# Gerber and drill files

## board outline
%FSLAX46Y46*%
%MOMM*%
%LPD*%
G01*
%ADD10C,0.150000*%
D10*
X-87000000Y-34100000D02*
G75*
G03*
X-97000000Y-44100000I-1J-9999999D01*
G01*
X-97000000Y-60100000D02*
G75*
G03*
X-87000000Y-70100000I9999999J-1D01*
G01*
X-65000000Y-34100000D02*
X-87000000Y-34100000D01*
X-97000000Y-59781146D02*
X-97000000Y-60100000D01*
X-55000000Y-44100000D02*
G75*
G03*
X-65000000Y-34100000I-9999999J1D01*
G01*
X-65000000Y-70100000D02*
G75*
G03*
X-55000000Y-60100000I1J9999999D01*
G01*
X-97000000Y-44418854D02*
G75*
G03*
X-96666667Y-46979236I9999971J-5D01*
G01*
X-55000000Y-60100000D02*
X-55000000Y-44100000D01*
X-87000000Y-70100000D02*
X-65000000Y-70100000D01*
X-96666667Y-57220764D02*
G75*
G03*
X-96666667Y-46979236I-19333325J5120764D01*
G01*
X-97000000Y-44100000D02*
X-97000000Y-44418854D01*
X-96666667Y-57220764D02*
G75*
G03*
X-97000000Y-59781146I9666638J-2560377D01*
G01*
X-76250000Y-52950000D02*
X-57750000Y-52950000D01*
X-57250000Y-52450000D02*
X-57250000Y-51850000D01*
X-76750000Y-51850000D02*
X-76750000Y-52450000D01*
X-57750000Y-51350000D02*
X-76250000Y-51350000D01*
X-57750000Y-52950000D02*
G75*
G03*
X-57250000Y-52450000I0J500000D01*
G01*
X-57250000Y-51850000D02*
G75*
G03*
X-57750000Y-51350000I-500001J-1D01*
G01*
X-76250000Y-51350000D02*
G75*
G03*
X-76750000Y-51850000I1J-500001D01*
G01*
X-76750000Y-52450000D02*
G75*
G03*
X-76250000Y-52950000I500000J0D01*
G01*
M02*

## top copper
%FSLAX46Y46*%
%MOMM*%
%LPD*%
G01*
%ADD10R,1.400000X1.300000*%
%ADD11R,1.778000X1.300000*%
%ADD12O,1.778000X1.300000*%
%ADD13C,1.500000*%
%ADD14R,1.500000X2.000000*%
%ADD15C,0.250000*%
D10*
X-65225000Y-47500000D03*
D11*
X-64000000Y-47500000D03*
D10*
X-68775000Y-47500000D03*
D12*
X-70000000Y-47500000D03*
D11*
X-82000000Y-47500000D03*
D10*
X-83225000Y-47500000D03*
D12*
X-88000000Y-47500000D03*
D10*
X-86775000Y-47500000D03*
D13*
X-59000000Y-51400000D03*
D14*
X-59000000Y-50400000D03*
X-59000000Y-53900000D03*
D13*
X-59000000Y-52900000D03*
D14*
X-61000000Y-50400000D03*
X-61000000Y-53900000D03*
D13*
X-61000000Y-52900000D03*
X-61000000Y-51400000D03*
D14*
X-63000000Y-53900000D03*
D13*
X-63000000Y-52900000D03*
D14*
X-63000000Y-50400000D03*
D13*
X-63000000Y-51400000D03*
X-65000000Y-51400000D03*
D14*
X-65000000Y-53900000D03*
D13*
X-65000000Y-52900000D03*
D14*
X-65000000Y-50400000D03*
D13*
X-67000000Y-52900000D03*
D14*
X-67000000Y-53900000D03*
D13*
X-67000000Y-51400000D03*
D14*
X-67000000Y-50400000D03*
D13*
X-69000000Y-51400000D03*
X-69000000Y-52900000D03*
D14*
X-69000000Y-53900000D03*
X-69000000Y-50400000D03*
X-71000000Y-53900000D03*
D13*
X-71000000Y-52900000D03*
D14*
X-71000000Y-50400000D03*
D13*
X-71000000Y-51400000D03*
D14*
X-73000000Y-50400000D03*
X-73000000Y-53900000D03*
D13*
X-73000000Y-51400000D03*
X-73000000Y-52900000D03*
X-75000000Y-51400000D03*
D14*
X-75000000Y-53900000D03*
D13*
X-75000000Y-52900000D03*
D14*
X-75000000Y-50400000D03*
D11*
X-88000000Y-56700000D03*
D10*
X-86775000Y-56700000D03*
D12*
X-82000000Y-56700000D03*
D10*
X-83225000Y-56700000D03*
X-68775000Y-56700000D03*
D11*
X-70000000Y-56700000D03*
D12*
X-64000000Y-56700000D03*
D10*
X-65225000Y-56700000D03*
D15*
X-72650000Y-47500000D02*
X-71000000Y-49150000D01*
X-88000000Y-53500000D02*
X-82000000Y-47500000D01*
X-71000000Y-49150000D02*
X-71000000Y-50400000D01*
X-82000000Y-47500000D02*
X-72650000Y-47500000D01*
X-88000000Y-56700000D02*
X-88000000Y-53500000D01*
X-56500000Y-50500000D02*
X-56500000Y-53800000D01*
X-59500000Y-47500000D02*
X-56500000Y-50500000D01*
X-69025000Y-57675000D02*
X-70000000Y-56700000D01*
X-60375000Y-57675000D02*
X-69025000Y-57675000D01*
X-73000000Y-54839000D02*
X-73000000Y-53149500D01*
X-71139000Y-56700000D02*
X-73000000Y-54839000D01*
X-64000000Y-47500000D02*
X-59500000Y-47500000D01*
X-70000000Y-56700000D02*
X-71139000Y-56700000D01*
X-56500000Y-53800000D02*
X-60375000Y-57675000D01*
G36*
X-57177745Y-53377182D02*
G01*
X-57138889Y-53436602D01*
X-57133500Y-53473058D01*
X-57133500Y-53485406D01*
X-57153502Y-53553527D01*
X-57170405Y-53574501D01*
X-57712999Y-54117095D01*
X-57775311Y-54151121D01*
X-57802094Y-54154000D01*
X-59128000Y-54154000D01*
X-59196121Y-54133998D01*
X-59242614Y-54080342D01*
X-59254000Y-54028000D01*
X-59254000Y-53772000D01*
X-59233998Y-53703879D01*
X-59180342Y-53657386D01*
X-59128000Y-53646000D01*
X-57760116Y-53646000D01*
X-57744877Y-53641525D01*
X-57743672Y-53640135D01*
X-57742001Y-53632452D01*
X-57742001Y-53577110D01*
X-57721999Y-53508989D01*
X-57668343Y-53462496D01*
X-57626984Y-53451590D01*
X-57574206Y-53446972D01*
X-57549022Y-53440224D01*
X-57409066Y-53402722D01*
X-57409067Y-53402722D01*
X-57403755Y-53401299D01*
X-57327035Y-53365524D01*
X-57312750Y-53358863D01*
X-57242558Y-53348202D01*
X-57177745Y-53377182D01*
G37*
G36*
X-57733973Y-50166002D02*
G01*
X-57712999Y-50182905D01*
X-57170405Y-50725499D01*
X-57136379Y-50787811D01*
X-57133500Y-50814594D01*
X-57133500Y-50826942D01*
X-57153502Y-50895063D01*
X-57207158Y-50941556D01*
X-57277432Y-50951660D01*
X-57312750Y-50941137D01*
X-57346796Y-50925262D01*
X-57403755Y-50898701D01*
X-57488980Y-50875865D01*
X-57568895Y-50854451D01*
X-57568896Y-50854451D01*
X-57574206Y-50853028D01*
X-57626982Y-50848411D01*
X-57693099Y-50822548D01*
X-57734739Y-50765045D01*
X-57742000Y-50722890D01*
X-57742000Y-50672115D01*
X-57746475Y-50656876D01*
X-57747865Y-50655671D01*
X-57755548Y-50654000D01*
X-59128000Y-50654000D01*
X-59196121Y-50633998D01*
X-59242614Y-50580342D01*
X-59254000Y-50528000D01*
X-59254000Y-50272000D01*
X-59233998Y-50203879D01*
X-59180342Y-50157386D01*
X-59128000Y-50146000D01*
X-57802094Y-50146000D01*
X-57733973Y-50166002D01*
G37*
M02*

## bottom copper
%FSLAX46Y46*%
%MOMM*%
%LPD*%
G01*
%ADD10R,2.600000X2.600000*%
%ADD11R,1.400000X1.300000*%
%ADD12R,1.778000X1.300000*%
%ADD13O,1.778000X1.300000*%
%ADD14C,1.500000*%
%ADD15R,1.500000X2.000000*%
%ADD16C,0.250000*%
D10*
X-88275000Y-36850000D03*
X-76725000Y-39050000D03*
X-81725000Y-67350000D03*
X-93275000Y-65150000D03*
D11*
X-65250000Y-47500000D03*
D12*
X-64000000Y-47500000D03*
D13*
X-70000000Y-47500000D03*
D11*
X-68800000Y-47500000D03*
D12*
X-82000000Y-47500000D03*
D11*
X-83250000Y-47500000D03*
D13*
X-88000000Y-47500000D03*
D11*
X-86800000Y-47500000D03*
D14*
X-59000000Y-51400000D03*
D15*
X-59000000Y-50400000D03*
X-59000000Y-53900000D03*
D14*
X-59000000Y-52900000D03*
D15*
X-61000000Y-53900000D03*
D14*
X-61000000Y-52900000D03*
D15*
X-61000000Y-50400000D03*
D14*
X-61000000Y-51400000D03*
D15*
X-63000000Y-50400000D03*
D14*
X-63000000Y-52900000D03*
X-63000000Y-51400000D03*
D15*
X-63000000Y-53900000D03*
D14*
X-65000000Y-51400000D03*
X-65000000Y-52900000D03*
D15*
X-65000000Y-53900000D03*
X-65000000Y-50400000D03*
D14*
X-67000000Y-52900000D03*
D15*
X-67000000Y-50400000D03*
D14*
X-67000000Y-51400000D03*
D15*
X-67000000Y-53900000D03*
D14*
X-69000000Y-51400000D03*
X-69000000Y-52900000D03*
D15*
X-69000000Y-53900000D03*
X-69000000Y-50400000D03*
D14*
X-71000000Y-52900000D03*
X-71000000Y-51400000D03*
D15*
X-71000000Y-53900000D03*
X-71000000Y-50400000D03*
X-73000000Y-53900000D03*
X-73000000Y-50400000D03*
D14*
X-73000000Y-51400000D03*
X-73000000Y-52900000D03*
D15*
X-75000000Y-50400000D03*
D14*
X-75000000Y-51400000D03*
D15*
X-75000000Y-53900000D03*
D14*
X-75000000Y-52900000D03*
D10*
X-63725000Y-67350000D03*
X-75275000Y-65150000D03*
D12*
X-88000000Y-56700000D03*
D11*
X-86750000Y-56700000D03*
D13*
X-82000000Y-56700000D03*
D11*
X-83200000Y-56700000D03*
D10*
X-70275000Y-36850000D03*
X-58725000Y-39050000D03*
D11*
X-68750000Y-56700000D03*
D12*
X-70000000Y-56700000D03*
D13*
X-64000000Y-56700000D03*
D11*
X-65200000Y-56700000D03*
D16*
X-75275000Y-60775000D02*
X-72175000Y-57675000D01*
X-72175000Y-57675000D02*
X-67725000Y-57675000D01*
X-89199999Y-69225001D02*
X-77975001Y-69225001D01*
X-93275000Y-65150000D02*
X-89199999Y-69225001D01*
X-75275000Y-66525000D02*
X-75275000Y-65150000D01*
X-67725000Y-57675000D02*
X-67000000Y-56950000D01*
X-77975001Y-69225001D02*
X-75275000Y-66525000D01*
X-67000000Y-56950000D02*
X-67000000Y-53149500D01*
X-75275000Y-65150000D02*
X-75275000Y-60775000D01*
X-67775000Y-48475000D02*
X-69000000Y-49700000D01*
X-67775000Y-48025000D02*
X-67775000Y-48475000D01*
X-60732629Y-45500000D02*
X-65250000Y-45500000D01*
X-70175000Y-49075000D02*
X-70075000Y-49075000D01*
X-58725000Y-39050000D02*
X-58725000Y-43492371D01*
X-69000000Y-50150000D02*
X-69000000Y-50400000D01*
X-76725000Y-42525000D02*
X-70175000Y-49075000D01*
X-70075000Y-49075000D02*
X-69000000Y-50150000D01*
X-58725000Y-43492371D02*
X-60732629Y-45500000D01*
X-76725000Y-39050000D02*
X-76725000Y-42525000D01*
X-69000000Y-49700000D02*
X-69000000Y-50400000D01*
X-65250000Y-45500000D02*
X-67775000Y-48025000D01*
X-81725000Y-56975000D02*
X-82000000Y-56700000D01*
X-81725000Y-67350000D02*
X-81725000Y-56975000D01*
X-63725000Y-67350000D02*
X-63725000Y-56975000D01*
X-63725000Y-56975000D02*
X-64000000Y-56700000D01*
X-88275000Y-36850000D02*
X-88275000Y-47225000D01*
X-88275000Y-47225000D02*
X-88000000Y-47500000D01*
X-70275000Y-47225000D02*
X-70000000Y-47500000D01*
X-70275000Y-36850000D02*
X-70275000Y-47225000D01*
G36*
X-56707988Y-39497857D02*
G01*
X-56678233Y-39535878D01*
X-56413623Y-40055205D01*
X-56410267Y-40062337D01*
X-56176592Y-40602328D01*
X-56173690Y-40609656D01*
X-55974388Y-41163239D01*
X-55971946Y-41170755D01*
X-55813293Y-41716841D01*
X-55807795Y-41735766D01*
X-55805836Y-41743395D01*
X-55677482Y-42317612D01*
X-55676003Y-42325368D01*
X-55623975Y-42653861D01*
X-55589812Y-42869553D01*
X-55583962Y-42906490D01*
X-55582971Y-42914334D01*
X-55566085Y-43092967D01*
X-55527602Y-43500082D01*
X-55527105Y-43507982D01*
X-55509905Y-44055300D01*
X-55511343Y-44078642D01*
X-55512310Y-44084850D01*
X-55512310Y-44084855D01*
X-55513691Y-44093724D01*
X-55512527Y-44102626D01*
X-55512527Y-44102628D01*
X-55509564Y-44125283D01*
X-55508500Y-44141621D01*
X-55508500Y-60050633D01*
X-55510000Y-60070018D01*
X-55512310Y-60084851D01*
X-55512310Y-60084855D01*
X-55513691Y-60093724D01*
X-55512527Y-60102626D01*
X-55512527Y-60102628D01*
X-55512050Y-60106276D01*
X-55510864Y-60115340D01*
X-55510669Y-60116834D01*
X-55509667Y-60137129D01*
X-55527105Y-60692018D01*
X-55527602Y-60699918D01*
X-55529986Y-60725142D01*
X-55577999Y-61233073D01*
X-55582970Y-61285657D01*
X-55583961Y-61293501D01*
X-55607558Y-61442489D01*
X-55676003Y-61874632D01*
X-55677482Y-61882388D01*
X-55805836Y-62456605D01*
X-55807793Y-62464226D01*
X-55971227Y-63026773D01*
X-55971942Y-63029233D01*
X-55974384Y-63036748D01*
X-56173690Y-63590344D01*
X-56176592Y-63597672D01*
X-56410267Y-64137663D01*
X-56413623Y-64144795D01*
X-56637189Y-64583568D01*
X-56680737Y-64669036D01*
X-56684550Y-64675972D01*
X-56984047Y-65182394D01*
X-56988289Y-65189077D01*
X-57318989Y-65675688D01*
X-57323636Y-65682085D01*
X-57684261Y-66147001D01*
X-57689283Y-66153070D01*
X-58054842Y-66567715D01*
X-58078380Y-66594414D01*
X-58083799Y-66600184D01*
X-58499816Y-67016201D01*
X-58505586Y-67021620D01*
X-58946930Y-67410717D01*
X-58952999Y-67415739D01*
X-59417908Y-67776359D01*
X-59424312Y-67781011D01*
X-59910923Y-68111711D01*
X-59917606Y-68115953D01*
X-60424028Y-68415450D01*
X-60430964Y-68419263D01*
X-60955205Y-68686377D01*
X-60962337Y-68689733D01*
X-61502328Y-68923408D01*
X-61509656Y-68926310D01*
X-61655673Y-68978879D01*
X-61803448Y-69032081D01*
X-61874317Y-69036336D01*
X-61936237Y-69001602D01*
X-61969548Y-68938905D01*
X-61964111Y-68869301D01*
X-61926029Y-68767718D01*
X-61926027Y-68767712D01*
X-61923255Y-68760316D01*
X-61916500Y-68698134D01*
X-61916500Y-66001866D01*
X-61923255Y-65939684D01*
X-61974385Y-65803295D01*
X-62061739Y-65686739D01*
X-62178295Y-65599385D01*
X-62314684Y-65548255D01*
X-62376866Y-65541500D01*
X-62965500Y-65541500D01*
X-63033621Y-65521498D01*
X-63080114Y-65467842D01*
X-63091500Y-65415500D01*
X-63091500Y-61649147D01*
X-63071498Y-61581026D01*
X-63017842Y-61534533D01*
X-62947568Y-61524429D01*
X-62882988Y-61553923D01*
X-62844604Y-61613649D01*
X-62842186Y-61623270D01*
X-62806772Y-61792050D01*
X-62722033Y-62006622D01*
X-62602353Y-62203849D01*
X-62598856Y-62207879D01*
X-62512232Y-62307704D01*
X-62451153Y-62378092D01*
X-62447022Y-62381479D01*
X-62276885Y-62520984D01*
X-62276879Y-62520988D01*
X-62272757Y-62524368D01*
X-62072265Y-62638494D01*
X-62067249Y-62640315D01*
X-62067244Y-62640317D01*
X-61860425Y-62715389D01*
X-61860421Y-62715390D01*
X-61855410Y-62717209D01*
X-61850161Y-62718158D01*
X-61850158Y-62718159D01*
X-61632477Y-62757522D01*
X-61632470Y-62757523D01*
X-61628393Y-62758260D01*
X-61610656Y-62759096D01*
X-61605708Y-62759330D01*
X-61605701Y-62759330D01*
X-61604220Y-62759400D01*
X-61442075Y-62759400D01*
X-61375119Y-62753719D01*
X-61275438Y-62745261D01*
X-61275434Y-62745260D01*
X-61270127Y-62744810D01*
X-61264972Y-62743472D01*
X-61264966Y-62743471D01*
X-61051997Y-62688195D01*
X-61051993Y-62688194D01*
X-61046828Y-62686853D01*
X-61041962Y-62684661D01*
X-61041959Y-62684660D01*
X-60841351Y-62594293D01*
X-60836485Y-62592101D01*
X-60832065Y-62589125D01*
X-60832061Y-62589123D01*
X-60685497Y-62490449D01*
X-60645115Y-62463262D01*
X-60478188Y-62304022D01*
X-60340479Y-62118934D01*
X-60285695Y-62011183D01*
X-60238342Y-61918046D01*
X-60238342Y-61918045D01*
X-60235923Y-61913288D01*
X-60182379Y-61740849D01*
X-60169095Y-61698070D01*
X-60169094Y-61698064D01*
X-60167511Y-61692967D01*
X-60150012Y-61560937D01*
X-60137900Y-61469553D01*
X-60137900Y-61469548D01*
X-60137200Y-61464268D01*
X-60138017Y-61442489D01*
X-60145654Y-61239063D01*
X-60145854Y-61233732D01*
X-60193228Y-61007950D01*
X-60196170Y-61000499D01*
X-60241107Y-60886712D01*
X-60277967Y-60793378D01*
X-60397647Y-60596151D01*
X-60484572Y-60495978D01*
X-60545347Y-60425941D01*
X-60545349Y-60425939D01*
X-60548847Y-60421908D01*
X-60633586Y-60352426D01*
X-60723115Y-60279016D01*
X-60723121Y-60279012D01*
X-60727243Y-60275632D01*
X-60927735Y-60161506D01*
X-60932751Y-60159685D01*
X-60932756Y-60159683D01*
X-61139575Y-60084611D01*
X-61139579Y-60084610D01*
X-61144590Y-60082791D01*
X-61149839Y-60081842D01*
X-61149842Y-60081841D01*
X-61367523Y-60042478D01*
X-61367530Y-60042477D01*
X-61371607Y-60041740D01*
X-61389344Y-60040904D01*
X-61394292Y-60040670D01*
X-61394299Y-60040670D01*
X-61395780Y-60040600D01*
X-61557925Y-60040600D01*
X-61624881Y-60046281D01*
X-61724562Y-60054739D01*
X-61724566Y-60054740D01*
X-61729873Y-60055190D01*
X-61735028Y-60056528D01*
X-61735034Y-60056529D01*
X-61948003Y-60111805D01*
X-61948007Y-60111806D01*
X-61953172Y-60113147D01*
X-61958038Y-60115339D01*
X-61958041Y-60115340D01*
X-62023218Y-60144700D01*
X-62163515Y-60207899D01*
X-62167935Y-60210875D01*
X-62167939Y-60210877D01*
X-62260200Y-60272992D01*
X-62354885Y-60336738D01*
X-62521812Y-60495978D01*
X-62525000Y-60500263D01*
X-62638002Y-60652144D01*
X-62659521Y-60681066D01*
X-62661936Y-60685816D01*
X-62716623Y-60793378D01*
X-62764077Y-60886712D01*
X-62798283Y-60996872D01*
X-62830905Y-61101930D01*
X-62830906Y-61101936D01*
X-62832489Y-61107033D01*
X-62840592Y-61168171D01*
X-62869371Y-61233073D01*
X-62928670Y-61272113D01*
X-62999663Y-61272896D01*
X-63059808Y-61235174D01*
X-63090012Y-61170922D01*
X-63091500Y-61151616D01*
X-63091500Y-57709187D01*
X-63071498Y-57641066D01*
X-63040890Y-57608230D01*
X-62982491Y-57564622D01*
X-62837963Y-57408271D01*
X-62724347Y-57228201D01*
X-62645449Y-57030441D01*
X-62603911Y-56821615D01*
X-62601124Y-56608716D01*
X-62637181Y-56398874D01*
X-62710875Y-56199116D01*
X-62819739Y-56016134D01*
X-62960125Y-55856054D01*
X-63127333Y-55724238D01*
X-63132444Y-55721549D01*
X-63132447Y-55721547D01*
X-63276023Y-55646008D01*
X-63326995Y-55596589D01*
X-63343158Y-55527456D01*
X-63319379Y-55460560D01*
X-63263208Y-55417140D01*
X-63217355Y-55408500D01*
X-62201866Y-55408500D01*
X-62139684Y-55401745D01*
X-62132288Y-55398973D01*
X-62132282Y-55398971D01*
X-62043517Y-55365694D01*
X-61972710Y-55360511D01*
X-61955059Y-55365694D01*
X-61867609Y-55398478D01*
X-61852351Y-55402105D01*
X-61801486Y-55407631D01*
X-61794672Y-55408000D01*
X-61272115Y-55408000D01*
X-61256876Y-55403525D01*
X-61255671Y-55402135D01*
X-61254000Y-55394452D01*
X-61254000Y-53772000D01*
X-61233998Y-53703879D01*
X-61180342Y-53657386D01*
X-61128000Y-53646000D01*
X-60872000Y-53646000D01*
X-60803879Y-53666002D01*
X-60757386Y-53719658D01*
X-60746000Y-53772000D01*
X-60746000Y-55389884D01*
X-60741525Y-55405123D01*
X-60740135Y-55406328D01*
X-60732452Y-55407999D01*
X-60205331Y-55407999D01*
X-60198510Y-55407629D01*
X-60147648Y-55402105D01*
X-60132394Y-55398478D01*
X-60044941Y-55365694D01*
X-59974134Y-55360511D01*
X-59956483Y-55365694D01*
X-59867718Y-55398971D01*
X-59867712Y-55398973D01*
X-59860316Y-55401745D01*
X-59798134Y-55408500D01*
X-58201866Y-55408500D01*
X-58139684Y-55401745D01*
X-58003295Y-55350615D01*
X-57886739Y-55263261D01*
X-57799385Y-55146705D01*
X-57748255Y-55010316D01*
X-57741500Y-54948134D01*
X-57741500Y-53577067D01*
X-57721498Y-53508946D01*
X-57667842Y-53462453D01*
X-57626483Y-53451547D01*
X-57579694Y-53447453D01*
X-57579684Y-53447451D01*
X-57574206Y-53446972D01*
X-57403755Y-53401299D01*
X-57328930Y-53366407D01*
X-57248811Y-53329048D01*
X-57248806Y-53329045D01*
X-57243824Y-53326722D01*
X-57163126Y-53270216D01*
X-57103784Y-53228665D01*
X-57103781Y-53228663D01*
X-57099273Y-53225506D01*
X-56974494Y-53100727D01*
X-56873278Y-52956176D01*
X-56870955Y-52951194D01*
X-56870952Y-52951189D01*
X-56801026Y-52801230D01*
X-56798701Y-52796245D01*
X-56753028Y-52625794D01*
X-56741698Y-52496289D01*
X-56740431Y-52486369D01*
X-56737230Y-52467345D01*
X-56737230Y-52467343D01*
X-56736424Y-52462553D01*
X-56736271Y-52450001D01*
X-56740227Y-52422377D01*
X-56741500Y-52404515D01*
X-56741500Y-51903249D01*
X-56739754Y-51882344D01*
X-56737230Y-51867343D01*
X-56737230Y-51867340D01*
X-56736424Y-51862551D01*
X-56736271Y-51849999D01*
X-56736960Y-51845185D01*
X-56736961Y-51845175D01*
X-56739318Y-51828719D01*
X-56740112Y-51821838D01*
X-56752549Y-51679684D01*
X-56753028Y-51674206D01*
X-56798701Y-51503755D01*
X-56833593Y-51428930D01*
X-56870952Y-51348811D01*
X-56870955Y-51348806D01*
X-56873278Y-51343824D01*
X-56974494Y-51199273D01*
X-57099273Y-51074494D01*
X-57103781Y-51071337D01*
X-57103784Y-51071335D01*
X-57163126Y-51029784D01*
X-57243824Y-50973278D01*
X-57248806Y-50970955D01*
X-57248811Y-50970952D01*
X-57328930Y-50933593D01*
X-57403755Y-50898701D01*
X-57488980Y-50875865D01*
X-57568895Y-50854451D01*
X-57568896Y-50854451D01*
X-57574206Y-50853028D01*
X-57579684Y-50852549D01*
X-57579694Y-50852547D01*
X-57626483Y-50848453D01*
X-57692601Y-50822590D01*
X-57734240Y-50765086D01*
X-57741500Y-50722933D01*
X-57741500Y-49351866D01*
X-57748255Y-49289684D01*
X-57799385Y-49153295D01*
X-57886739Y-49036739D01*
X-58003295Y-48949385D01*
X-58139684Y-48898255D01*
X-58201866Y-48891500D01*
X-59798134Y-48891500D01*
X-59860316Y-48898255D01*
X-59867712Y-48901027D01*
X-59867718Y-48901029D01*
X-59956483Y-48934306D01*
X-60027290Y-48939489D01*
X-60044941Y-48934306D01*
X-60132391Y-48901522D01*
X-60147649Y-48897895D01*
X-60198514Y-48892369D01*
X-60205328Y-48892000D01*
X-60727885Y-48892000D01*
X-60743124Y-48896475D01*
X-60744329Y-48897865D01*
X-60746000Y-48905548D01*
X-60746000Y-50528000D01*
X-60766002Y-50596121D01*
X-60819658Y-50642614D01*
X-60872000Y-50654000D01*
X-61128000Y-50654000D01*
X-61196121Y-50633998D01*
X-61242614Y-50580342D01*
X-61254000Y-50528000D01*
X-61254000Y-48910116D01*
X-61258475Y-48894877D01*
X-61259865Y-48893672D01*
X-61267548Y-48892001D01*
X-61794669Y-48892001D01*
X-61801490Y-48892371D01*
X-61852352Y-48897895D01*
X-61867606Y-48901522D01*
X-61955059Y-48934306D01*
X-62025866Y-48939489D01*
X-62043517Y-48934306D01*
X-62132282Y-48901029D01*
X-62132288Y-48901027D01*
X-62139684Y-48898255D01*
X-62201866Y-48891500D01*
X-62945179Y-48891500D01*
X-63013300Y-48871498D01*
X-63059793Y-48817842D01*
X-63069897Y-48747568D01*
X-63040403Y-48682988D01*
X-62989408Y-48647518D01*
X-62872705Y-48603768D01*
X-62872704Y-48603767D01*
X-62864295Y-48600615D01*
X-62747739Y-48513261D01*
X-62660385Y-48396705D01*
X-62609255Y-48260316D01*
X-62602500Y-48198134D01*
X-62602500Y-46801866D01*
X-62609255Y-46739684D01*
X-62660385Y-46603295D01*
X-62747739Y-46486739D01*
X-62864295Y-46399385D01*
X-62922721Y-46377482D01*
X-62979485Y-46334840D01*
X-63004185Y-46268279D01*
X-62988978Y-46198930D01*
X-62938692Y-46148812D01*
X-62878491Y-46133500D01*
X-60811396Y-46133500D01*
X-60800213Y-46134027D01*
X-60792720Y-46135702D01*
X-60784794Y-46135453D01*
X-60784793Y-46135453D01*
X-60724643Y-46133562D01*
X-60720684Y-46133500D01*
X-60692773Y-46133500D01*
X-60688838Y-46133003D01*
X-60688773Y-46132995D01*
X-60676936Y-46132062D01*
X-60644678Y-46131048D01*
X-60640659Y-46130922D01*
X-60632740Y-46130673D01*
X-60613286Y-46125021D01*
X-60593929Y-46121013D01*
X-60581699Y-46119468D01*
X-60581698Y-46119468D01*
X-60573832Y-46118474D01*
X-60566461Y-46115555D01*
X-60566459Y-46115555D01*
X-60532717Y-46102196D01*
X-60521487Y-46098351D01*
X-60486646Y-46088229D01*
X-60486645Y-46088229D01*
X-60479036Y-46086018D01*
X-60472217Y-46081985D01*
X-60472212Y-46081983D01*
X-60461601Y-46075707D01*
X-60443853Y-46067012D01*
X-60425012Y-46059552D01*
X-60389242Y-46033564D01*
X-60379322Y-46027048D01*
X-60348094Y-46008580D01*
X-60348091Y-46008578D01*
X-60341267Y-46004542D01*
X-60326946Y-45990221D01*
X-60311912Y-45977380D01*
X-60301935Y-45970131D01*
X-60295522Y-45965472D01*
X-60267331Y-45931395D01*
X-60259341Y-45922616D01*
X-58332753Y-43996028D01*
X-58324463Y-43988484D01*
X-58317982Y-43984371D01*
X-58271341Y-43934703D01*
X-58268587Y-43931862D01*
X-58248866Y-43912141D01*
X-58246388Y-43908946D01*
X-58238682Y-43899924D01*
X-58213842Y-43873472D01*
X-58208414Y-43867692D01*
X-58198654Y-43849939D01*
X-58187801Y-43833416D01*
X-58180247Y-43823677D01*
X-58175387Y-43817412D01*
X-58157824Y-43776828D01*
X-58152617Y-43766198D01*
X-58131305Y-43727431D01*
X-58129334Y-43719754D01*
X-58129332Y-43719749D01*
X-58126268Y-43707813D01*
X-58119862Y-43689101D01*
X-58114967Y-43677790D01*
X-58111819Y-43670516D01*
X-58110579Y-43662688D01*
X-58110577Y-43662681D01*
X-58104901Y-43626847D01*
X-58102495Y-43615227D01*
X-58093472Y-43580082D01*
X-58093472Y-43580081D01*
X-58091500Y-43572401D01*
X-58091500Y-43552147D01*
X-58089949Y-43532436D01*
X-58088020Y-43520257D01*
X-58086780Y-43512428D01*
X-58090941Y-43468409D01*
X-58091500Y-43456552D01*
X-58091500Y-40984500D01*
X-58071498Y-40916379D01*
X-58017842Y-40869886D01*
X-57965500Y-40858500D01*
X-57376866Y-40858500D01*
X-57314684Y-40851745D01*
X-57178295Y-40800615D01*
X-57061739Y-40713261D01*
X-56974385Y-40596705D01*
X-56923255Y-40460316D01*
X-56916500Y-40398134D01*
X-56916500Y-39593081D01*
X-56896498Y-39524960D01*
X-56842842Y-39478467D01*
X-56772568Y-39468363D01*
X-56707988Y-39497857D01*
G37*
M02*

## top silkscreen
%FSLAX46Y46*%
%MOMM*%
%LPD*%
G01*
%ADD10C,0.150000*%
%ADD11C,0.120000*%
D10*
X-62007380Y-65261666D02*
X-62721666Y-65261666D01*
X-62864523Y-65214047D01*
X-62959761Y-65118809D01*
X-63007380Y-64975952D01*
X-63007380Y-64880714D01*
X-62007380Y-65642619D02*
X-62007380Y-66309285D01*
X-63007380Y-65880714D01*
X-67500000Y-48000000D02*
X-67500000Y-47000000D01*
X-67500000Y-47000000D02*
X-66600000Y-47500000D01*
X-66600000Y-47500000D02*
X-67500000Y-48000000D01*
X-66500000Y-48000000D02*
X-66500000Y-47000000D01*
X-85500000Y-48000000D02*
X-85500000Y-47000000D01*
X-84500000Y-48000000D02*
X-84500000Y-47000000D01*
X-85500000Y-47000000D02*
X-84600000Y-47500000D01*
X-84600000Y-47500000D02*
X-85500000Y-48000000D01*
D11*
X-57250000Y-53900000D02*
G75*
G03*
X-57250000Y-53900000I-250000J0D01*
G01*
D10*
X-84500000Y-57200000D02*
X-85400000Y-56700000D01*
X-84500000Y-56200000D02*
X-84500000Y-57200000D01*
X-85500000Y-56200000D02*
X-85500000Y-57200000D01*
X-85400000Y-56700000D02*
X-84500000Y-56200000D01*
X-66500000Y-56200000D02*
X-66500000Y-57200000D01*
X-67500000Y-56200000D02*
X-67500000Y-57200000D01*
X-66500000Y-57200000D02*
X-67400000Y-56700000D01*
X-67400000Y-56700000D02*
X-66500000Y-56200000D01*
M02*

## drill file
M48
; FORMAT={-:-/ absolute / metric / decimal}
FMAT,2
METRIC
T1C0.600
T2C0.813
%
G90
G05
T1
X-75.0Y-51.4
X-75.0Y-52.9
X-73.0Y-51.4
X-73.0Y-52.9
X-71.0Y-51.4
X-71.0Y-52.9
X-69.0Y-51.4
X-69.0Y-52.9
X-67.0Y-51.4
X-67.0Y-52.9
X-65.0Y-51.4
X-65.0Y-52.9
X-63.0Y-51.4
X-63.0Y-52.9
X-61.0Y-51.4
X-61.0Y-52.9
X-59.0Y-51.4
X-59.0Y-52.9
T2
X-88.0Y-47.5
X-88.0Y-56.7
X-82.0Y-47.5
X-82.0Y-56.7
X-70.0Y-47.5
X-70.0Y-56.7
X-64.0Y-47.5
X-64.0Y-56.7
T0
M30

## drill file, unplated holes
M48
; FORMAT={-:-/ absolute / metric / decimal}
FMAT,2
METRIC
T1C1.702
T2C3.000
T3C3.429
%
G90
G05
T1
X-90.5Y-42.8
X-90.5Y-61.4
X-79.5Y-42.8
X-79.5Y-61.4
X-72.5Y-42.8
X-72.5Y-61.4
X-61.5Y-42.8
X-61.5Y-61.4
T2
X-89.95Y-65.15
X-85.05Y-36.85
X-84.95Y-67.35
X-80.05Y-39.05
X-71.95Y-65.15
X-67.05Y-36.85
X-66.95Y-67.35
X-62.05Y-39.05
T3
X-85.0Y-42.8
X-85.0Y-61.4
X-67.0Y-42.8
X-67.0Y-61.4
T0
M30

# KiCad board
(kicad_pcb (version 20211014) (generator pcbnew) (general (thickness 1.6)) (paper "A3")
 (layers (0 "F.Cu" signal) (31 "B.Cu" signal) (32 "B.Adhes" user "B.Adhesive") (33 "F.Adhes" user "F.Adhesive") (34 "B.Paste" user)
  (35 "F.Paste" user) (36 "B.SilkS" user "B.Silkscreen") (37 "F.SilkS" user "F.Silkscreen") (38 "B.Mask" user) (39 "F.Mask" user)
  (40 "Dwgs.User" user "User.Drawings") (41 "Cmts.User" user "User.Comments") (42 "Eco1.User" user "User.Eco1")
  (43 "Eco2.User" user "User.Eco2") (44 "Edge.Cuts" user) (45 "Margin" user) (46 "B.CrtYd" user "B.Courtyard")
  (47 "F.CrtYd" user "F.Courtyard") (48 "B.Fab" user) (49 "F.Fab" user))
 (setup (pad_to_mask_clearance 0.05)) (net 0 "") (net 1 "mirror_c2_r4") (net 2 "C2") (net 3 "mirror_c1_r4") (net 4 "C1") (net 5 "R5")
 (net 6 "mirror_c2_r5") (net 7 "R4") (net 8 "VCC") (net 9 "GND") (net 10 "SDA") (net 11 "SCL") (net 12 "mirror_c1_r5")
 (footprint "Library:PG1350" (layer "F.Cu") (at -85 42.8)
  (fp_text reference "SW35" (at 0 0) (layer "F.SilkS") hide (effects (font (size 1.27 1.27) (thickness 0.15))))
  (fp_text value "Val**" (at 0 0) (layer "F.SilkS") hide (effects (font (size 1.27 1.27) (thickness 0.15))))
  (pad "" np_thru_hole circle (at -0.05 -5.95 270) (size 3 3) (drill 3) (layers *.Cu *.Mask))
  (pad "" np_thru_hole circle (at 4.95 -3.75 270) (size 3 3) (drill 3) (layers *.Cu *.Mask))
  (pad "" np_thru_hole circle (at 0 0) (size 3.429 3.429) (drill 3.429) (layers *.Cu *.Mask))
  (pad "" np_thru_hole circle (at 5.5 0) (size 1.7018 1.7018) (drill 1.7018) (layers *.Cu *.Mask))
  (pad "" np_thru_hole circle (at -5.5 0) (size 1.7018 1.7018) (drill 1.7018) (layers *.Cu *.Mask))
  (pad "1" smd rect (at -3.275 -5.95) (size 2.6 2.6) (layers "B.Cu" "B.Paste" "B.Mask") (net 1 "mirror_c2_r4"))
  (pad "2" smd rect (at 8.275 -3.75) (size 2.6 2.6) (layers "B.Cu" "B.Paste" "B.Mask") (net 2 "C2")))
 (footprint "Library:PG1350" (layer "F.Cu") (at -85 61.4 180)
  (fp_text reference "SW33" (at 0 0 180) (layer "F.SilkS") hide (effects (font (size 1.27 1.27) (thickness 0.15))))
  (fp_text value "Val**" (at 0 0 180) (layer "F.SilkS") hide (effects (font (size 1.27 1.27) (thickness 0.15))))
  (pad "" np_thru_hole circle (at 0 0 180) (size 3.429 3.429) (drill 3.429) (layers *.Cu *.Mask))
  (pad "" np_thru_hole circle (at 5.5 0 180) (size 1.7018 1.7018) (drill 1.7018) (layers *.Cu *.Mask))
  (pad "" np_thru_hole circle (at -0.05 -5.95 90) (size 3 3) (drill 3) (layers *.Cu *.Mask))
  (pad "" np_thru_hole circle (at 4.95 -3.75 90) (size 3 3) (drill 3) (layers *.Cu *.Mask))
  (pad "" np_thru_hole circle (at -5.5 0 180) (size 1.7018 1.7018) (drill 1.7018) (layers *.Cu *.Mask))
  (pad "1" smd rect (at -3.275 -5.95 180) (size 2.6 2.6) (layers "B.Cu" "B.Paste" "B.Mask") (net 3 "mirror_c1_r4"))
  (pad "2" smd rect (at 8.275 -3.75 180) (size 2.6 2.6) (layers "B.Cu" "B.Paste" "B.Mask") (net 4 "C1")))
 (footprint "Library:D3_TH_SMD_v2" (layer "F.Cu") (at -67 47.5 180) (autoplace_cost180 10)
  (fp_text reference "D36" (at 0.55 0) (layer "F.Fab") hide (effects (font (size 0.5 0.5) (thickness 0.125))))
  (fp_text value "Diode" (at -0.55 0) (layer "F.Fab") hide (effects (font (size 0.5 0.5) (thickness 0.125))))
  (fp_line (start 0.5 -0.5) (end 0.5 0.5) (layer "F.SilkS") (width 0.15))
  (fp_line (start 0.5 0.5) (end -0.4 0) (layer "F.SilkS") (width 0.15))
  (fp_line (start -0.4 0) (end 0.5 -0.5) (layer "F.SilkS") (width 0.15))
  (fp_line (start -0.5 -0.5) (end -0.5 0.5) (layer "F.SilkS") (width 0.15))
  (pad "1" smd rect (at -1.775 0) (size 1.4 1.3) (layers "F.Cu" "F.Paste" "F.Mask") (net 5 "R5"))
  (pad "1" smd rect (at -1.75 0 180) (size 1.4 1.3) (layers "B.Cu" "B.Paste" "B.Mask") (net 5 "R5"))
  (pad "1" thru_hole rect (at -3 0 180) (size 1.778 1.3) (drill 0.8128) (layers *.Cu "B.Mask") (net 5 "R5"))
  (pad "2" smd rect (at 1.775 0) (size 1.4 1.3) (layers "F.Cu" "F.Paste" "F.Mask") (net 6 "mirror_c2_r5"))
  (pad "2" thru_hole oval (at 3 0 180) (size 1.778 1.3) (drill 0.8128) (layers *.Cu "B.Mask") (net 6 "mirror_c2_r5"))
  (pad "2" smd rect (at 1.8 0 180) (size 1.4 1.3) (layers "B.Cu" "B.Paste" "B.Mask") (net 6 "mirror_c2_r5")))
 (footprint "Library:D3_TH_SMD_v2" (layer "F.Cu") (at -85 47.5 180) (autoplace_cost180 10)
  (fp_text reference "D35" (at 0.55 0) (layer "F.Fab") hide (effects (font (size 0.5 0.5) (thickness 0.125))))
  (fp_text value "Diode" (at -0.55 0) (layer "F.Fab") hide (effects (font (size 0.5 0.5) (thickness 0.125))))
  (fp_line (start 0.5 -0.5) (end 0.5 0.5) (layer "F.SilkS") (width 0.15))
  (fp_line (start -0.5 -0.5) (end -0.5 0.5) (layer "F.SilkS") (width 0.15))
  (fp_line (start 0.5 0.5) (end -0.4 0) (layer "F.SilkS") (width 0.15))
  (fp_line (start -0.4 0) (end 0.5 -0.5) (layer "F.SilkS") (width 0.15))
  (pad "1" thru_hole rect (at -3 0 180) (size 1.778 1.3) (drill 0.8128) (layers *.Cu "B.Mask") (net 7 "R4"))
  (pad "1" smd rect (at -1.775 0) (size 1.4 1.3) (layers "F.Cu" "F.Paste" "F.Mask") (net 7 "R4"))
  (pad "1" smd rect (at -1.75 0 180) (size 1.4 1.3) (layers "B.Cu" "B.Paste" "B.Mask") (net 7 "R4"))
  (pad "2" thru_hole oval (at 3 0 180) (size 1.778 1.3) (drill 0.8128) (layers *.Cu "B.Mask") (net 1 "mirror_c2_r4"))
  (pad "2" smd rect (at 1.775 0) (size 1.4 1.3) (layers "F.Cu" "F.Paste" "F.Mask") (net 1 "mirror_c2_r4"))
  (pad "2" smd rect (at 1.8 0 180) (size 1.4 1.3) (layers "B.Cu" "B.Paste" "B.Mask") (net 1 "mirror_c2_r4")))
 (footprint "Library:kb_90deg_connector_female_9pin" (layer "F.Cu") (at -67 52.15 -90)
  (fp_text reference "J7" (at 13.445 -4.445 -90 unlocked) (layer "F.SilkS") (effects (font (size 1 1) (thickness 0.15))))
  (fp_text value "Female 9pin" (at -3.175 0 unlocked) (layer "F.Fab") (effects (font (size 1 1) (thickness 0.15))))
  (fp_circle (center 1.75 -9.5) (end 2 -9.5) (layer "F.SilkS") (width 0.12) (fill none))
  (fp_line (start 0.8 9.25) (end 0.8 -9.25) (layer "Edge.Cuts") (width 0.15))
  (fp_line (start 0.3 -9.75) (end -0.3 -9.75) (layer "Edge.Cuts") (width 0.15))
  (fp_line (start -0.3 9.75) (end 0.3 9.75) (layer "Edge.Cuts") (width 0.15))
  (fp_line (start -0.8 -9.25) (end -0.8 9.25) (layer "Edge.Cuts") (width 0.15))
  (fp_arc (start 0.3 -9.75) (mid 0.653553 -9.603553) (end 0.8 -9.25) (layer "Edge.Cuts") (width 0.15))
  (fp_arc (start -0.8 -9.25) (mid -0.653553 -9.603553) (end -0.3 -9.75) (layer "Edge.Cuts") (width 0.15))
  (fp_arc (start -0.3 9.75) (mid -0.653553 9.603553) (end -0.8 9.25) (layer "Edge.Cuts") (width 0.15))
  (fp_arc (start 0.8 9.25) (mid 0.653553 9.603553) (end 0.3 9.75) (layer "Edge.Cuts") (width 0.15))
  (pad "1" thru_hole circle (at -0.75 -8 270) (size 1.5 1.5) (drill 0.6) (layers *.Cu) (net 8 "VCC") (zone_connect 2))
  (pad "1" smd rect (at -1.75 -8 90) (size 2 1.5) (layers "B.Cu" "B.Paste" "B.Mask") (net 8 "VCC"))
  (pad "1" smd rect (at -1.75 -8 90) (size 2 1.5) (layers "F.Cu" "F.Paste" "F.Mask") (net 8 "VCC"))
  (pad "1" smd rect (at 1.75 -8 90) (size 2 1.5) (layers "B.Cu" "B.Paste" "B.Mask") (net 8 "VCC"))
  (pad "1" smd rect (at 1.75 -8 90) (size 2 1.5) (layers "F.Cu" "F.Paste" "F.Mask") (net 8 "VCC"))
  (pad "1" thru_hole circle (at 0.75 -8 270) (size 1.5 1.5) (drill 0.6) (layers *.Cu) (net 8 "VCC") (zone_connect 2))
  (pad "2" smd rect (at 1.75 -6 90) (size 2 1.5) (layers "B.Cu" "B.Paste" "B.Mask") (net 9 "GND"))
  (pad "2" smd rect (at -1.75 -6 90) (size 2 1.5) (layers "F.Cu" "F.Paste" "F.Mask") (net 9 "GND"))
  (pad "2" smd rect (at 1.75 -6 90) (size 2 1.5) (layers "F.Cu" "F.Paste" "F.Mask") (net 9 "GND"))
  (pad "2" thru_hole circle (at 0.75 -6 270) (size 1.5 1.5) (drill 0.6) (layers *.Cu) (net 9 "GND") (zone_connect 2))
  (pad "2" smd rect (at -1.75 -6 90) (size 2 1.5) (layers "B.Cu" "B.Paste" "B.Mask") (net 9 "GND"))
  (pad "2" thru_hole circle (at -0.75 -6 270) (size 1.5 1.5) (drill 0.6) (layers *.Cu) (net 9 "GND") (zone_connect 2))
  (pad "3" smd rect (at -1.75 -4 90) (size 2 1.5) (layers "B.Cu" "B.Paste" "B.Mask") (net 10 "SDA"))
  (pad "3" smd rect (at 1.75 -4 90) (size 2 1.5) (layers "F.Cu" "F.Paste" "F.Mask") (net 10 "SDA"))
  (pad "3" thru_hole circle (at 0.75 -4 270) (size 1.5 1.5) (drill 0.6) (layers *.Cu) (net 10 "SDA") (zone_connect 2))
  (pad "3" smd rect (at -1.75 -4 90) (size 2 1.5) (layers "F.Cu" "F.Paste" "F.Mask") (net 10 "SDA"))
  (pad "3" thru_hole circle (at -0.75 -4 270) (size 1.5 1.5) (drill 0.6) (layers *.Cu) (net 10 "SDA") (zone_connect 2))
  (pad "3" smd rect (at 1.75 -4 90) (size 2 1.5) (layers "B.Cu" "B.Paste" "B.Mask") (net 10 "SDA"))
  (pad "4" thru_hole circle (at -0.75 -2 270) (size 1.5 1.5) (drill 0.6) (layers *.Cu) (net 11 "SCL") (zone_connect 2))
  (pad "4" smd rect (at 1.75 -2 90) (size 2 1.5) (layers "F.Cu" "F.Paste" "F.Mask") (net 11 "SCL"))
  (pad "4" thru_hole circle (at 0.75 -2 270) (size 1.5 1.5) (drill 0.6) (layers *.Cu) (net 11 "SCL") (zone_connect 2))
  (pad "4" smd rect (at 1.75 -2 90) (size 2 1.5) (layers "B.Cu" "B.Paste" "B.Mask") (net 11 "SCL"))
  (pad "4" smd rect (at -1.75 -2 90) (size 2 1.5) (layers "F.Cu" "F.Paste" "F.Mask") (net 11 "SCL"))
  (pad "4" smd rect (at -1.75 -2 90) (size 2 1.5) (layers "B.Cu" "B.Paste" "B.Mask") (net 11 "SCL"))
  (pad "5" thru_hole circle (at 0.75 0 270) (size 1.5 1.5) (drill 0.6) (layers *.Cu) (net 4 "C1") (zone_connect 2))
  (pad "5" smd rect (at -1.75 0 90) (size 2 1.5) (layers "B.Cu" "B.Paste" "B.Mask") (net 4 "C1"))
  (pad "5" smd rect (at 1.75 0 90) (size 2 1.5) (layers "F.Cu" "F.Paste" "F.Mask") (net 4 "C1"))
  (pad "5" thru_hole circle (at -0.75 0 270) (size 1.5 1.5) (drill 0.6) (layers *.Cu) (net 4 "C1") (zone_connect 2))
  (pad "5" smd rect (at 1.75 0 90) (size 2 1.5) (layers "B.Cu" "B.Paste" "B.Mask") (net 4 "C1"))
  (pad "5" smd rect (at -1.75 0 90) (size 2 1.5) (layers "F.Cu" "F.Paste" "F.Mask") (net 4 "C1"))
  (pad "6" thru_hole circle (at -0.75 2 270) (size 1.5 1.5) (drill 0.6) (layers *.Cu) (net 2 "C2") (zone_connect 2))
  (pad "6" thru_hole circle (at 0.75 2 270) (size 1.5 1.5) (drill 0.6) (layers *.Cu) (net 2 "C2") (zone_connect 2))
  (pad "6" smd rect (at 1.75 2 90) (size 2 1.5) (layers "F.Cu" "F.Paste" "F.Mask") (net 2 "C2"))
  (pad "6" smd rect (at -1.75 2 90) (size 2 1.5) (layers "F.Cu" "F.Paste" "F.Mask") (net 2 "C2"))
  (pad "6" smd rect (at 1.75 2 90) (size 2 1.5) (layers "B.Cu" "B.Paste" "B.Mask") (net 2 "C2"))
  (pad "6" smd rect (at -1.75 2 90) (size 2 1.5) (layers "B.Cu" "B.Paste" "B.Mask") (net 2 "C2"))
  (pad "7" smd rect (at 1.75 4 90) (size 2 1.5) (layers "F.Cu" "F.Paste" "F.Mask") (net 7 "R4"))
  (pad "7" thru_hole circle (at 0.75 4 270) (size 1.5 1.5) (drill 0.6) (layers *.Cu) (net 7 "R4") (zone_connect 2))
  (pad "7" smd rect (at -1.75 4 90) (size 2 1.5) (layers "F.Cu" "F.Paste" "F.Mask") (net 7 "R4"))
  (pad "7" thru_hole circle (at -0.75 4 270) (size 1.5 1.5) (drill 0.6) (layers *.Cu) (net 7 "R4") (zone_connect 2))
  (pad "7" smd rect (at 1.75 4 90) (size 2 1.5) (layers "B.Cu" "B.Paste" "B.Mask") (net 7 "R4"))
  (pad "7" smd rect (at -1.75 4 90) (size 2 1.5) (layers "B.Cu" "B.Paste" "B.Mask") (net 7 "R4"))
  (pad "8" smd rect (at 1.75 6 90) (size 2 1.5) (layers "B.Cu" "B.Paste" "B.Mask") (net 5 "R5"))
  (pad "8" smd rect (at -1.75 6 90) (size 2 1.5) (layers "F.Cu" "F.Paste" "F.Mask") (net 5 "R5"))
  (pad "8" smd rect (at -1.75 6 90) (size 2 1.5) (layers "B.Cu" "B.Paste" "B.Mask") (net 5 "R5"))
  (pad "8" smd rect (at 1.75 6 90) (size 2 1.5) (layers "F.Cu" "F.Paste" "F.Mask") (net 5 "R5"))
  (pad "8" thru_hole circle (at -0.75 6 270) (size 1.5 1.5) (drill 0.6) (layers *.Cu) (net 5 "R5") (zone_connect 2))
  (pad "8" thru_hole circle (at 0.75 6 270) (size 1.5 1.5) (drill 0.6) (layers *.Cu) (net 5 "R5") (zone_connect 2))
  (pad "9" smd rect (at -1.75 8 90) (size 2 1.5) (layers "B.Cu" "B.Paste" "B.Mask"))
  (pad "9" thru_hole circle (at -0.75 8 270) (size 1.5 1.5) (drill 0.6) (layers *.Cu) (zone_connect 2))
  (pad "9" smd rect (at 1.75 8 90) (size 2 1.5) (layers "F.Cu" "F.Paste" "F.Mask"))
  (pad "9" smd rect (at 1.75 8 90) (size 2 1.5) (layers "B.Cu" "B.Paste" "B.Mask"))
  (pad "9" thru_hole circle (at 0.75 8 270) (size 1.5 1.5) (drill 0.6) (layers *.Cu) (zone_connect 2))
  (pad "9" smd rect (at -1.75 8 90) (size 2 1.5) (layers "F.Cu" "F.Paste" "F.Mask")))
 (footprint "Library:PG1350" (layer "F.Cu") (at -67 61.4 180)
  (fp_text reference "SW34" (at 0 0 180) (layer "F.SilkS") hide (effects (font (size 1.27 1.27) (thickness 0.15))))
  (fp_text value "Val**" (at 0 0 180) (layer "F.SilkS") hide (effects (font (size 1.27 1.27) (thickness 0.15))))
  (pad "" np_thru_hole circle (at -5.5 0 180) (size 1.7018 1.7018) (drill 1.7018) (layers *.Cu *.Mask))
  (pad "" np_thru_hole circle (at 0 0 180) (size 3.429 3.429) (drill 3.429) (layers *.Cu *.Mask))
  (pad "" np_thru_hole circle (at 5.5 0 180) (size 1.7018 1.7018) (drill 1.7018) (layers *.Cu *.Mask))
  (pad "" np_thru_hole circle (at -0.05 -5.95 90) (size 3 3) (drill 3) (layers *.Cu *.Mask))
  (pad "" np_thru_hole circle (at 4.95 -3.75 90) (size 3 3) (drill 3) (layers *.Cu *.Mask))
  (pad "1" smd rect (at -3.275 -5.95 180) (size 2.6 2.6) (layers "B.Cu" "B.Paste" "B.Mask") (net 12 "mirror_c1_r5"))
  (pad "2" smd rect (at 8.275 -3.75 180) (size 2.6 2.6) (layers "B.Cu" "B.Paste" "B.Mask") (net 4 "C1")))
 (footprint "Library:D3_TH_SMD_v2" (layer "F.Cu") (at -85 56.7) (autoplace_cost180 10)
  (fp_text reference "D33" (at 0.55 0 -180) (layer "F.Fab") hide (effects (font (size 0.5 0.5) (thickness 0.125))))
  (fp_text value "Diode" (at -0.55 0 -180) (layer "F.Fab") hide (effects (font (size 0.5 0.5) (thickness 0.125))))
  (fp_line (start 0.5 0.5) (end -0.4 0) (layer "F.SilkS") (width 0.15))
  (fp_line (start 0.5 -0.5) (end 0.5 0.5) (layer "F.SilkS") (width 0.15))
  (fp_line (start -0.5 -0.5) (end -0.5 0.5) (layer "F.SilkS") (width 0.15))
  (fp_line (start -0.4 0) (end 0.5 -0.5) (layer "F.SilkS") (width 0.15))
  (pad "1" thru_hole rect (at -3 0) (size 1.778 1.3) (drill 0.8128) (layers *.Cu "B.Mask") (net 7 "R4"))
  (pad "1" smd rect (at -1.75 0) (size 1.4 1.3) (layers "B.Cu" "B.Paste" "B.Mask") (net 7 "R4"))
  (pad "1" smd rect (at -1.775 0 180) (size 1.4 1.3) (layers "F.Cu" "F.Paste" "F.Mask") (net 7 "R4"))
  (pad "2" thru_hole oval (at 3 0) (size 1.778 1.3) (drill 0.8128) (layers *.Cu "B.Mask") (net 3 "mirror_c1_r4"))
  (pad "2" smd rect (at 1.8 0) (size 1.4 1.3) (layers "B.Cu" "B.Paste" "B.Mask") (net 3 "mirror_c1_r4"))
  (pad "2" smd rect (at 1.775 0 180) (size 1.4 1.3) (layers "F.Cu" "F.Paste" "F.Mask") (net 3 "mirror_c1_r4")))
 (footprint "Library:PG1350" (layer "F.Cu") (at -67 42.8)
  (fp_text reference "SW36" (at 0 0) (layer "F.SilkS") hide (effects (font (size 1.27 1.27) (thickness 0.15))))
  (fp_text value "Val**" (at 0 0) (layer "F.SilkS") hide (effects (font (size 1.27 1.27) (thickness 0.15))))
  (pad "" np_thru_hole circle (at 4.95 -3.75 270) (size 3 3) (drill 3) (layers *.Cu *.Mask))
  (pad "" np_thru_hole circle (at -5.5 0) (size 1.7018 1.7018) (drill 1.7018) (layers *.Cu *.Mask))
  (pad "" np_thru_hole circle (at 0 0) (size 3.429 3.429) (drill 3.429) (layers *.Cu *.Mask))
  (pad "" np_thru_hole circle (at -0.05 -5.95 270) (size 3 3) (drill 3) (layers *.Cu *.Mask))
  (pad "" np_thru_hole circle (at 5.5 0) (size 1.7018 1.7018) (drill 1.7018) (layers *.Cu *.Mask))
  (pad "1" smd rect (at -3.275 -5.95) (size 2.6 2.6) (layers "B.Cu" "B.Paste" "B.Mask") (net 6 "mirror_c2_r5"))
  (pad "2" smd rect (at 8.275 -3.75) (size 2.6 2.6) (layers "B.Cu" "B.Paste" "B.Mask") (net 2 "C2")))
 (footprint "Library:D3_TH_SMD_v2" (layer "F.Cu") (at -67 56.7) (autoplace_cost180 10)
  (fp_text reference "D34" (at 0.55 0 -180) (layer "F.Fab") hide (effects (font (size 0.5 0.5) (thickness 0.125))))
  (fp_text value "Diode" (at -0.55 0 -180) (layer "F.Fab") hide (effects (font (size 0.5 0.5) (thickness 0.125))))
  (fp_line (start 0.5 -0.5) (end 0.5 0.5) (layer "F.SilkS") (width 0.15))
  (fp_line (start -0.5 -0.5) (end -0.5 0.5) (layer "F.SilkS") (width 0.15))
  (fp_line (start 0.5 0.5) (end -0.4 0) (layer "F.SilkS") (width 0.15))
  (fp_line (start -0.4 0) (end 0.5 -0.5) (layer "F.SilkS") (width 0.15))
  (pad "1" smd rect (at -1.775 0 180) (size 1.4 1.3) (layers "F.Cu" "F.Paste" "F.Mask") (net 5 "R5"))
  (pad "1" smd rect (at -1.75 0) (size 1.4 1.3) (layers "B.Cu" "B.Paste" "B.Mask") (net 5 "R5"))
  (pad "1" thru_hole rect (at -3 0) (size 1.778 1.3) (drill 0.8128) (layers *.Cu "B.Mask") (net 5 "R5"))
  (pad "2" thru_hole oval (at 3 0) (size 1.778 1.3) (drill 0.8128) (layers *.Cu "B.Mask") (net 12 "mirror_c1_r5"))
  (pad "2" smd rect (at 1.775 0 180) (size 1.4 1.3) (layers "F.Cu" "F.Paste" "F.Mask") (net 12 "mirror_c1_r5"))
  (pad "2" smd rect (at 1.8 0) (size 1.4 1.3) (layers "B.Cu" "B.Paste" "B.Mask") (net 12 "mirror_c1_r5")))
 (gr_arc (start -97 44.1) (mid -94.071068 37.028932) (end -87 34.1) (layer "Edge.Cuts") (width 0.15))
 (gr_arc (start -87 70.1) (mid -94.071068 67.171068) (end -97 60.1) (layer "Edge.Cuts") (width 0.15))
 (gr_line (start -65 34.1) (end -87 34.1) (layer "Edge.Cuts") (width 0.15))
 (gr_line (start -97 59.781146) (end -97 60.1) (layer "Edge.Cuts") (width 0.15))
 (gr_arc (start -65 34.1) (mid -57.928932 37.028932) (end -55 44.1) (layer "Edge.Cuts") (width 0.15))
 (gr_arc (start -55 60.1) (mid -57.928932 67.171068) (end -65 70.1) (layer "Edge.Cuts") (width 0.15))
 (gr_arc (start -96.666667 46.979236) (mid -96.916317 45.709848) (end -97 44.418854) (layer "Edge.Cuts") (width 0.15))
 (gr_line (start -55 60.1) (end -55 44.1) (layer "Edge.Cuts") (width 0.15))
 (gr_line (start -87 70.1) (end -65 70.1) (layer "Edge.Cuts") (width 0.15))
 (gr_arc (start -96.666667 46.979236) (mid -96 52.1) (end -96.666667 57.220764) (layer "Edge.Cuts") (width 0.15))
 (gr_line (start -97 44.1) (end -97 44.418854) (layer "Edge.Cuts") (width 0.15))
 (gr_arc (start -97 59.781146) (mid -96.916317 58.490152) (end -96.666667 57.220764) (layer "Edge.Cuts") (width 0.15))
 (segment (start -75.275 60.775) (end -72.175 57.675) (width 0.25) (layer "B.Cu") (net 4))
 (segment (start -72.175 57.675) (end -67.725 57.675) (width 0.25) (layer "B.Cu") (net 4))
 (segment (start -89.199999 69.225001) (end -77.975001 69.225001) (width 0.25) (layer "B.Cu") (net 4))
 (segment (start -93.275 65.15) (end -89.199999 69.225001) (width 0.25) (layer "B.Cu") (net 4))
 (segment (start -75.275 66.525) (end -75.275 65.15) (width 0.25) (layer "B.Cu") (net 4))
 (segment (start -67.725 57.675) (end -67 56.95) (width 0.25) (layer "B.Cu") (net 4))
 (segment (start -77.975001 69.225001) (end -75.275 66.525) (width 0.25) (layer "B.Cu") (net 4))
 (segment (start -67 56.95) (end -67 53.1495) (width 0.25) (layer "B.Cu") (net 4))
 (segment (start -75.275 65.15) (end -75.275 60.775) (width 0.25) (layer "B.Cu") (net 4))
 (segment (start -67.775 48.475) (end -69 49.7) (width 0.25) (layer "B.Cu") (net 2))
 (segment (start -67.775 48.025) (end -67.775 48.475) (width 0.25) (layer "B.Cu") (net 2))
 (segment (start -60.732629 45.5) (end -65.25 45.5) (width 0.25) (layer "B.Cu") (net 2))
 (segment (start -70.175 49.075) (end -70.075 49.075) (width 0.25) (layer "B.Cu") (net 2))
 (segment (start -58.725 39.05) (end -58.725 43.492371) (width 0.25) (layer "B.Cu") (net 2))
 (segment (start -69 50.15) (end -69 50.4) (width 0.25) (layer "B.Cu") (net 2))
 (segment (start -76.725 42.525) (end -70.175 49.075) (width 0.25) (layer "B.Cu") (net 2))
 (segment (start -70.075 49.075) (end -69 50.15) (width 0.25) (layer "B.Cu") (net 2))
 (segment (start -58.725 43.492371) (end -60.732629 45.5) (width 0.25) (layer "B.Cu") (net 2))
 (segment (start -76.725 39.05) (end -76.725 42.525) (width 0.25) (layer "B.Cu") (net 2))
 (segment (start -69 49.7) (end -69 50.4) (width 0.25) (layer "B.Cu") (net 2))
 (segment (start -65.25 45.5) (end -67.775 48.025) (width 0.25) (layer "B.Cu") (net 2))
 (segment (start -72.65 47.5) (end -71 49.15) (width 0.25) (layer "F.Cu") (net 7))
 (segment (start -88 53.5) (end -82 47.5) (width 0.25) (layer "F.Cu") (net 7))
 (segment (start -71 49.15) (end -71 50.4) (width 0.25) (layer "F.Cu") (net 7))
 (segment (start -82 47.5) (end -72.65 47.5) (width 0.25) (layer "F.Cu") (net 7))
 (segment (start -88 56.7) (end -88 53.5) (width 0.25) (layer "F.Cu") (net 7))
 (segment (start -81.725 56.975) (end -82 56.7) (width 0.25) (layer "B.Cu") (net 3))
 (segment (start -81.725 67.35) (end -81.725 56.975) (width 0.25) (layer "B.Cu") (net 3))
 (segment (start -63.725 67.35) (end -63.725 56.975) (width 0.25) (layer "B.Cu") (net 12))
 (segment (start -63.725 56.975) (end -64 56.7) (width 0.25) (layer "B.Cu") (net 12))
 (segment (start -56.5 50.5) (end -56.5 53.8) (width 0.25) (layer "F.Cu") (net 5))
 (segment (start -59.5 47.5) (end -56.5 50.5) (width 0.25) (layer "F.Cu") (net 5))
 (segment (start -69.025 57.675) (end -70 56.7) (width 0.25) (layer "F.Cu") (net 5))
 (segment (start -60.375 57.675) (end -69.025 57.675) (width 0.25) (layer "F.Cu") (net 5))
 (segment (start -73 54.839) (end -73 53.1495) (width 0.25) (layer "F.Cu") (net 5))
 (segment (start -71.139 56.7) (end -73 54.839) (width 0.25) (layer "F.Cu") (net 5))
 (segment (start -64 47.5) (end -59.5 47.5) (width 0.25) (layer "F.Cu") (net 5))
 (segment (start -70 56.7) (end -71.139 56.7) (width 0.25) (layer "F.Cu") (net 5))
 (segment (start -56.5 53.8) (end -60.375 57.675) (width 0.25) (layer "F.Cu") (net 5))
 (segment (start -88.275 36.85) (end -88.275 47.225) (width 0.25) (layer "B.Cu") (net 1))
 (segment (start -88.275 47.225) (end -88 47.5) (width 0.25) (layer "B.Cu") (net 1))
 (segment (start -70.275 47.225) (end -70 47.5) (width 0.25) (layer "B.Cu") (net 6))
 (segment (start -70.275 36.85) (end -70.275 47.225) (width 0.25) (layer "B.Cu") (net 6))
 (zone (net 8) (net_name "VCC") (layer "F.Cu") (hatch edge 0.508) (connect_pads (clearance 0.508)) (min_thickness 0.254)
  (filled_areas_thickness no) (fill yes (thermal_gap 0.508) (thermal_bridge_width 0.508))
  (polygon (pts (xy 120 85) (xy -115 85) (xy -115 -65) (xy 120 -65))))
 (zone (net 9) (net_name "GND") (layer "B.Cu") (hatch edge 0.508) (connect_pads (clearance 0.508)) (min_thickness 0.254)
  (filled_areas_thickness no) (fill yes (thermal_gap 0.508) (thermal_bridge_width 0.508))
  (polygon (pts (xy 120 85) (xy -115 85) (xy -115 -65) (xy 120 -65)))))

